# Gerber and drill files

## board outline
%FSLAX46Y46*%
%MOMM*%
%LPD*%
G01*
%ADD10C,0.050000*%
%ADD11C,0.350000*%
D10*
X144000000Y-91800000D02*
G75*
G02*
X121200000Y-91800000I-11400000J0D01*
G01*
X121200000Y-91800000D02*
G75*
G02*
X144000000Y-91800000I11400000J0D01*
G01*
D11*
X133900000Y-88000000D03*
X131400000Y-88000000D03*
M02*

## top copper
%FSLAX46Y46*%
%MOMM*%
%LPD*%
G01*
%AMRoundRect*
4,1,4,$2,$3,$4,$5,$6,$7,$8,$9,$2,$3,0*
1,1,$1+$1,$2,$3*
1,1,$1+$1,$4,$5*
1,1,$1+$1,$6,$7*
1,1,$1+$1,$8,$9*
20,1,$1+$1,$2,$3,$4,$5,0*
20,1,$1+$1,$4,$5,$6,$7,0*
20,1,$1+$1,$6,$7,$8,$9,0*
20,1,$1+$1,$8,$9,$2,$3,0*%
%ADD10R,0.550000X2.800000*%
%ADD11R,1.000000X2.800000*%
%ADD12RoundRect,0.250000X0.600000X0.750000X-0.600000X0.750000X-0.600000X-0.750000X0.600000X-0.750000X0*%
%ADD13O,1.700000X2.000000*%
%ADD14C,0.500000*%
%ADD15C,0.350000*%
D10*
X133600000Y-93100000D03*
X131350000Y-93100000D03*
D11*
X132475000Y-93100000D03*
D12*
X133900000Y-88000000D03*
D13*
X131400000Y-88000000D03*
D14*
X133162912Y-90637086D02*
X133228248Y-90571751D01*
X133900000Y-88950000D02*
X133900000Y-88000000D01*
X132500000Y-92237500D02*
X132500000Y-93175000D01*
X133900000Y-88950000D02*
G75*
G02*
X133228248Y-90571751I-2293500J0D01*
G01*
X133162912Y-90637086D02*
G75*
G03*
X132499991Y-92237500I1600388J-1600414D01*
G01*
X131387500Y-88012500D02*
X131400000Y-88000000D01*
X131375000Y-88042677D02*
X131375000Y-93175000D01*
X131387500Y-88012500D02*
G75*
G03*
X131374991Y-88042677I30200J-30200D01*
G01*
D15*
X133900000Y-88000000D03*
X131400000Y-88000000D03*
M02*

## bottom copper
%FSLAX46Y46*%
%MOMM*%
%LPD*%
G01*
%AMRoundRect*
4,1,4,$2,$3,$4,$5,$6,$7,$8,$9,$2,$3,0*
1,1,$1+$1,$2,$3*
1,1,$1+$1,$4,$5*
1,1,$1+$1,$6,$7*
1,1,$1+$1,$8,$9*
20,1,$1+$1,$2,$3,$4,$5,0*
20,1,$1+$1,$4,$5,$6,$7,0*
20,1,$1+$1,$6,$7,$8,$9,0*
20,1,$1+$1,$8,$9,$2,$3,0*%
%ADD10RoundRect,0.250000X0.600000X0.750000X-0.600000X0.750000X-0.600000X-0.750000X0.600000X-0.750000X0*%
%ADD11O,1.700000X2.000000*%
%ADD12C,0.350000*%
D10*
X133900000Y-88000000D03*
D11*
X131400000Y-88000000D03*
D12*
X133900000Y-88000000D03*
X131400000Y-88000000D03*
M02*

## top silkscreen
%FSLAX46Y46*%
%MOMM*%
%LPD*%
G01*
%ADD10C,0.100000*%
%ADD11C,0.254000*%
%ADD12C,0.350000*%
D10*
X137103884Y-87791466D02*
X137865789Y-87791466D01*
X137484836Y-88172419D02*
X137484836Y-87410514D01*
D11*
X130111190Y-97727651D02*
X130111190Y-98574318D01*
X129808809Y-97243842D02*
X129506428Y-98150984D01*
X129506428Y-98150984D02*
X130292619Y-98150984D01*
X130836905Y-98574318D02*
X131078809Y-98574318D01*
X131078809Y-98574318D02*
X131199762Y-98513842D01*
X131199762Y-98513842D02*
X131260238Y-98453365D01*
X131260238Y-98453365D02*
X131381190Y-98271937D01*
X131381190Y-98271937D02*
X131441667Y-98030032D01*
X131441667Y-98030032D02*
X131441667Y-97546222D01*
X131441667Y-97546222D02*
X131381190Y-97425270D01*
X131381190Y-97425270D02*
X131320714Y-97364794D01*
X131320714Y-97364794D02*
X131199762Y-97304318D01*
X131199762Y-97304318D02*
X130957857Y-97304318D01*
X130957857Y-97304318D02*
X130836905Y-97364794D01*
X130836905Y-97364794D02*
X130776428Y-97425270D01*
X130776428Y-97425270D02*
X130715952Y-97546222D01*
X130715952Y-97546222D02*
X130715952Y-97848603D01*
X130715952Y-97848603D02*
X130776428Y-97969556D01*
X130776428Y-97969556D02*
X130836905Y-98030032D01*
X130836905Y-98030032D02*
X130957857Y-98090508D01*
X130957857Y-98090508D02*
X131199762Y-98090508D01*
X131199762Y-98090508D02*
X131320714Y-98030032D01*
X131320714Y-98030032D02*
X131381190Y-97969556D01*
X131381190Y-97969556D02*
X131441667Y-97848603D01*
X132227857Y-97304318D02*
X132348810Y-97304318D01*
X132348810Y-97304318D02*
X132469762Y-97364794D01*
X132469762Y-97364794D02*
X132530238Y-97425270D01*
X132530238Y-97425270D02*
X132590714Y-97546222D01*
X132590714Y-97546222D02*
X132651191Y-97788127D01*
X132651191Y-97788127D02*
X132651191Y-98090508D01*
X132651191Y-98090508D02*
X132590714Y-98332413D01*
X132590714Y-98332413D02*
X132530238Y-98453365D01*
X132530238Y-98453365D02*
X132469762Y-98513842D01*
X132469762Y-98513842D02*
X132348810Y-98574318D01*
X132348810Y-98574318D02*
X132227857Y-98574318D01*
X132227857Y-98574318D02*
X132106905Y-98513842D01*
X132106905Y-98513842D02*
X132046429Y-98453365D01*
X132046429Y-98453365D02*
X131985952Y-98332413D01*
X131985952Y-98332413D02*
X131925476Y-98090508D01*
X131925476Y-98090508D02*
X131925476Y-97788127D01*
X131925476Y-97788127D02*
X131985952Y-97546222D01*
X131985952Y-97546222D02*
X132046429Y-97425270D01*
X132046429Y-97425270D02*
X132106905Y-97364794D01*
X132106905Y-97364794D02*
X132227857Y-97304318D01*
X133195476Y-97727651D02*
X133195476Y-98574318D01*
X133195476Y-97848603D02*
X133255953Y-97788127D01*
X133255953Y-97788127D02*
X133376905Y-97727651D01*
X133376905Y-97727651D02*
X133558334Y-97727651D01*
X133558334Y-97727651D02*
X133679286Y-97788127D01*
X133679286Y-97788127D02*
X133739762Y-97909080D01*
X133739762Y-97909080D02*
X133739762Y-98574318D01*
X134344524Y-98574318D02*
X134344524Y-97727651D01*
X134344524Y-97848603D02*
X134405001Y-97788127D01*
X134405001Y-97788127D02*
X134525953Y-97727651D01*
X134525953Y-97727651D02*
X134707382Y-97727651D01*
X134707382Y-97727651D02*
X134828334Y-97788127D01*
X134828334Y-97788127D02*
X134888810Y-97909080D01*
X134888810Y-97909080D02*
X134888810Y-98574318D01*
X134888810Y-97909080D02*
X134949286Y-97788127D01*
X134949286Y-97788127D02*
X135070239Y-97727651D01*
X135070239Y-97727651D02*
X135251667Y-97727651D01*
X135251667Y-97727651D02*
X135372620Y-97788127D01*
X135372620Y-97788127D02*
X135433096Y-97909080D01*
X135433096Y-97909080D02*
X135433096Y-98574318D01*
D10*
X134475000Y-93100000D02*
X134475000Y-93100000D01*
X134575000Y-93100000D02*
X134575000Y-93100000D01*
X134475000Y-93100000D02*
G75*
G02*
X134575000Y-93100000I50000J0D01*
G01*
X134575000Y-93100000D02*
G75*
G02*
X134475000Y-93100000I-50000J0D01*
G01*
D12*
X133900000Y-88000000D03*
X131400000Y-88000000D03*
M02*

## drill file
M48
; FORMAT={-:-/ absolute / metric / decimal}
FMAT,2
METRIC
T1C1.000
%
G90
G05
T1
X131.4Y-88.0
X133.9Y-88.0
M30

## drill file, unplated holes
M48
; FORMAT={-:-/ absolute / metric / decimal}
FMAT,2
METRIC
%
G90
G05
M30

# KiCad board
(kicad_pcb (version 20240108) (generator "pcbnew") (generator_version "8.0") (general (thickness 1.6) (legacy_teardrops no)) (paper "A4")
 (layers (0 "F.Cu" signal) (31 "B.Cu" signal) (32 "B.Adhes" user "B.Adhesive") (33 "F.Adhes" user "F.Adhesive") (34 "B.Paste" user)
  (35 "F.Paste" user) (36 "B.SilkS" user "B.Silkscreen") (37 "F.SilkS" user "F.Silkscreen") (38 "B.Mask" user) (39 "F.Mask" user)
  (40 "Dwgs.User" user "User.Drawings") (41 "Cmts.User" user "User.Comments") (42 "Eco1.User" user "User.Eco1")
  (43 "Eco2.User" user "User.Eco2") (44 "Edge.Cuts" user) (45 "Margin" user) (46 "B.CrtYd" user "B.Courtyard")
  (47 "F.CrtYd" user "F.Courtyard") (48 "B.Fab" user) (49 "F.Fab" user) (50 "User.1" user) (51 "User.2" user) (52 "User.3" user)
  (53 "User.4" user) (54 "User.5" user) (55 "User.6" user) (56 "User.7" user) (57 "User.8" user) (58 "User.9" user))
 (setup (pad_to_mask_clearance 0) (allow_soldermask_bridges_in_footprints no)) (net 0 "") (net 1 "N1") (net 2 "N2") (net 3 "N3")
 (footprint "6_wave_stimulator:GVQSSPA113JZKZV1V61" (layer "F.Cu") (at 132.475 93.1 90)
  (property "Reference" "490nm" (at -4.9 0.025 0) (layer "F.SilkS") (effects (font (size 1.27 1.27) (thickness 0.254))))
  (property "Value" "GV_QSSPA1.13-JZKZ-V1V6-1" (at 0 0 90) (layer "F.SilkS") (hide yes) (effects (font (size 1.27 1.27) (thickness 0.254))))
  (fp_line (start 0 2) (end 0 2) (stroke (width 0.1) (type solid)) (layer "F.SilkS"))
  (fp_line (start 0 2.1) (end 0 2.1) (stroke (width 0.1) (type solid)) (layer "F.SilkS"))
  (fp_arc (start 0 2) (mid 0.05 2.05) (end 0 2.1) (stroke (width 0.1) (type solid)) (layer "F.SilkS"))
  (fp_arc (start 0 2.1) (mid -0.05 2.05) (end 0 2) (stroke (width 0.1) (type solid)) (layer "F.SilkS"))
  (pad "1" smd rect (at 0 1.125 180) (size 0.55 2.8) (layers "F.Cu" "F.Paste" "F.Mask") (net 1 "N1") (thermal_bridge_angle 45))
  (pad "2" smd rect (at 0 -1.125 180) (size 0.55 2.8) (layers "F.Cu" "F.Paste" "F.Mask") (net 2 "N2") (thermal_bridge_angle 45))
  (pad "3" smd rect (at 0 0 180) (size 1 2.8) (layers "F.Cu" "F.Paste" "F.Mask") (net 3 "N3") (thermal_bridge_angle 45)))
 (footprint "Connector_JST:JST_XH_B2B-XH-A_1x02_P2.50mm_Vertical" (layer "B.Cu") (at 133.9 88 180)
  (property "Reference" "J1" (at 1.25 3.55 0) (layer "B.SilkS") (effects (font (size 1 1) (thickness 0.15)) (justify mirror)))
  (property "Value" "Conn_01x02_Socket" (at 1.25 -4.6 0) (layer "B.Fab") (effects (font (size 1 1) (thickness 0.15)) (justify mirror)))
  (pad "1" thru_hole roundrect (at 0 0 180) (size 1.7 2) (drill 1) (layers "*.Cu" "*.Mask") (remove_unused_layers no)
   (roundrect_rratio 0.147059) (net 3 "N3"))
  (pad "2" thru_hole oval (at 2.5 0 180) (size 1.7 2) (drill 1) (layers "*.Cu" "*.Mask") (remove_unused_layers no) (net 2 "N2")))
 (gr_circle (center 132.6 91.8) (end 144 91.8) (stroke (width 0.05) (type default)) (fill none) (layer "Edge.Cuts"))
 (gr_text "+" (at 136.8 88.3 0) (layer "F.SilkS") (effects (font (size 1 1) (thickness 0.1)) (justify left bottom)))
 (segment (start 133.162912 90.637086) (end 133.228248 90.571751) (width 0.5) (layer "F.Cu") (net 3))
 (segment (start 133.9 88.95) (end 133.9 88) (width 0.5) (layer "F.Cu") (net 3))
 (segment (start 132.5 92.2375) (end 132.5 93.175) (width 0.5) (layer "F.Cu") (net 3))
 (arc (start 133.9 88.95) (mid 133.725417 89.827685) (end 133.228248 90.571751) (width 0.5) (layer "F.Cu") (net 3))
 (arc (start 133.162912 90.637086) (mid 132.672285 91.371362) (end 132.5 92.2375) (width 0.5) (layer "F.Cu") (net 3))
 (segment (start 131.3875 88.0125) (end 131.4 88) (width 0.5) (layer "F.Cu") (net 2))
 (segment (start 131.375 88.042677) (end 131.375 93.175) (width 0.5) (layer "F.Cu") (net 2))
 (arc (start 131.3875 88.0125) (mid 131.378248 88.026345) (end 131.375 88.042677) (width 0.5) (layer "F.Cu") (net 2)))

